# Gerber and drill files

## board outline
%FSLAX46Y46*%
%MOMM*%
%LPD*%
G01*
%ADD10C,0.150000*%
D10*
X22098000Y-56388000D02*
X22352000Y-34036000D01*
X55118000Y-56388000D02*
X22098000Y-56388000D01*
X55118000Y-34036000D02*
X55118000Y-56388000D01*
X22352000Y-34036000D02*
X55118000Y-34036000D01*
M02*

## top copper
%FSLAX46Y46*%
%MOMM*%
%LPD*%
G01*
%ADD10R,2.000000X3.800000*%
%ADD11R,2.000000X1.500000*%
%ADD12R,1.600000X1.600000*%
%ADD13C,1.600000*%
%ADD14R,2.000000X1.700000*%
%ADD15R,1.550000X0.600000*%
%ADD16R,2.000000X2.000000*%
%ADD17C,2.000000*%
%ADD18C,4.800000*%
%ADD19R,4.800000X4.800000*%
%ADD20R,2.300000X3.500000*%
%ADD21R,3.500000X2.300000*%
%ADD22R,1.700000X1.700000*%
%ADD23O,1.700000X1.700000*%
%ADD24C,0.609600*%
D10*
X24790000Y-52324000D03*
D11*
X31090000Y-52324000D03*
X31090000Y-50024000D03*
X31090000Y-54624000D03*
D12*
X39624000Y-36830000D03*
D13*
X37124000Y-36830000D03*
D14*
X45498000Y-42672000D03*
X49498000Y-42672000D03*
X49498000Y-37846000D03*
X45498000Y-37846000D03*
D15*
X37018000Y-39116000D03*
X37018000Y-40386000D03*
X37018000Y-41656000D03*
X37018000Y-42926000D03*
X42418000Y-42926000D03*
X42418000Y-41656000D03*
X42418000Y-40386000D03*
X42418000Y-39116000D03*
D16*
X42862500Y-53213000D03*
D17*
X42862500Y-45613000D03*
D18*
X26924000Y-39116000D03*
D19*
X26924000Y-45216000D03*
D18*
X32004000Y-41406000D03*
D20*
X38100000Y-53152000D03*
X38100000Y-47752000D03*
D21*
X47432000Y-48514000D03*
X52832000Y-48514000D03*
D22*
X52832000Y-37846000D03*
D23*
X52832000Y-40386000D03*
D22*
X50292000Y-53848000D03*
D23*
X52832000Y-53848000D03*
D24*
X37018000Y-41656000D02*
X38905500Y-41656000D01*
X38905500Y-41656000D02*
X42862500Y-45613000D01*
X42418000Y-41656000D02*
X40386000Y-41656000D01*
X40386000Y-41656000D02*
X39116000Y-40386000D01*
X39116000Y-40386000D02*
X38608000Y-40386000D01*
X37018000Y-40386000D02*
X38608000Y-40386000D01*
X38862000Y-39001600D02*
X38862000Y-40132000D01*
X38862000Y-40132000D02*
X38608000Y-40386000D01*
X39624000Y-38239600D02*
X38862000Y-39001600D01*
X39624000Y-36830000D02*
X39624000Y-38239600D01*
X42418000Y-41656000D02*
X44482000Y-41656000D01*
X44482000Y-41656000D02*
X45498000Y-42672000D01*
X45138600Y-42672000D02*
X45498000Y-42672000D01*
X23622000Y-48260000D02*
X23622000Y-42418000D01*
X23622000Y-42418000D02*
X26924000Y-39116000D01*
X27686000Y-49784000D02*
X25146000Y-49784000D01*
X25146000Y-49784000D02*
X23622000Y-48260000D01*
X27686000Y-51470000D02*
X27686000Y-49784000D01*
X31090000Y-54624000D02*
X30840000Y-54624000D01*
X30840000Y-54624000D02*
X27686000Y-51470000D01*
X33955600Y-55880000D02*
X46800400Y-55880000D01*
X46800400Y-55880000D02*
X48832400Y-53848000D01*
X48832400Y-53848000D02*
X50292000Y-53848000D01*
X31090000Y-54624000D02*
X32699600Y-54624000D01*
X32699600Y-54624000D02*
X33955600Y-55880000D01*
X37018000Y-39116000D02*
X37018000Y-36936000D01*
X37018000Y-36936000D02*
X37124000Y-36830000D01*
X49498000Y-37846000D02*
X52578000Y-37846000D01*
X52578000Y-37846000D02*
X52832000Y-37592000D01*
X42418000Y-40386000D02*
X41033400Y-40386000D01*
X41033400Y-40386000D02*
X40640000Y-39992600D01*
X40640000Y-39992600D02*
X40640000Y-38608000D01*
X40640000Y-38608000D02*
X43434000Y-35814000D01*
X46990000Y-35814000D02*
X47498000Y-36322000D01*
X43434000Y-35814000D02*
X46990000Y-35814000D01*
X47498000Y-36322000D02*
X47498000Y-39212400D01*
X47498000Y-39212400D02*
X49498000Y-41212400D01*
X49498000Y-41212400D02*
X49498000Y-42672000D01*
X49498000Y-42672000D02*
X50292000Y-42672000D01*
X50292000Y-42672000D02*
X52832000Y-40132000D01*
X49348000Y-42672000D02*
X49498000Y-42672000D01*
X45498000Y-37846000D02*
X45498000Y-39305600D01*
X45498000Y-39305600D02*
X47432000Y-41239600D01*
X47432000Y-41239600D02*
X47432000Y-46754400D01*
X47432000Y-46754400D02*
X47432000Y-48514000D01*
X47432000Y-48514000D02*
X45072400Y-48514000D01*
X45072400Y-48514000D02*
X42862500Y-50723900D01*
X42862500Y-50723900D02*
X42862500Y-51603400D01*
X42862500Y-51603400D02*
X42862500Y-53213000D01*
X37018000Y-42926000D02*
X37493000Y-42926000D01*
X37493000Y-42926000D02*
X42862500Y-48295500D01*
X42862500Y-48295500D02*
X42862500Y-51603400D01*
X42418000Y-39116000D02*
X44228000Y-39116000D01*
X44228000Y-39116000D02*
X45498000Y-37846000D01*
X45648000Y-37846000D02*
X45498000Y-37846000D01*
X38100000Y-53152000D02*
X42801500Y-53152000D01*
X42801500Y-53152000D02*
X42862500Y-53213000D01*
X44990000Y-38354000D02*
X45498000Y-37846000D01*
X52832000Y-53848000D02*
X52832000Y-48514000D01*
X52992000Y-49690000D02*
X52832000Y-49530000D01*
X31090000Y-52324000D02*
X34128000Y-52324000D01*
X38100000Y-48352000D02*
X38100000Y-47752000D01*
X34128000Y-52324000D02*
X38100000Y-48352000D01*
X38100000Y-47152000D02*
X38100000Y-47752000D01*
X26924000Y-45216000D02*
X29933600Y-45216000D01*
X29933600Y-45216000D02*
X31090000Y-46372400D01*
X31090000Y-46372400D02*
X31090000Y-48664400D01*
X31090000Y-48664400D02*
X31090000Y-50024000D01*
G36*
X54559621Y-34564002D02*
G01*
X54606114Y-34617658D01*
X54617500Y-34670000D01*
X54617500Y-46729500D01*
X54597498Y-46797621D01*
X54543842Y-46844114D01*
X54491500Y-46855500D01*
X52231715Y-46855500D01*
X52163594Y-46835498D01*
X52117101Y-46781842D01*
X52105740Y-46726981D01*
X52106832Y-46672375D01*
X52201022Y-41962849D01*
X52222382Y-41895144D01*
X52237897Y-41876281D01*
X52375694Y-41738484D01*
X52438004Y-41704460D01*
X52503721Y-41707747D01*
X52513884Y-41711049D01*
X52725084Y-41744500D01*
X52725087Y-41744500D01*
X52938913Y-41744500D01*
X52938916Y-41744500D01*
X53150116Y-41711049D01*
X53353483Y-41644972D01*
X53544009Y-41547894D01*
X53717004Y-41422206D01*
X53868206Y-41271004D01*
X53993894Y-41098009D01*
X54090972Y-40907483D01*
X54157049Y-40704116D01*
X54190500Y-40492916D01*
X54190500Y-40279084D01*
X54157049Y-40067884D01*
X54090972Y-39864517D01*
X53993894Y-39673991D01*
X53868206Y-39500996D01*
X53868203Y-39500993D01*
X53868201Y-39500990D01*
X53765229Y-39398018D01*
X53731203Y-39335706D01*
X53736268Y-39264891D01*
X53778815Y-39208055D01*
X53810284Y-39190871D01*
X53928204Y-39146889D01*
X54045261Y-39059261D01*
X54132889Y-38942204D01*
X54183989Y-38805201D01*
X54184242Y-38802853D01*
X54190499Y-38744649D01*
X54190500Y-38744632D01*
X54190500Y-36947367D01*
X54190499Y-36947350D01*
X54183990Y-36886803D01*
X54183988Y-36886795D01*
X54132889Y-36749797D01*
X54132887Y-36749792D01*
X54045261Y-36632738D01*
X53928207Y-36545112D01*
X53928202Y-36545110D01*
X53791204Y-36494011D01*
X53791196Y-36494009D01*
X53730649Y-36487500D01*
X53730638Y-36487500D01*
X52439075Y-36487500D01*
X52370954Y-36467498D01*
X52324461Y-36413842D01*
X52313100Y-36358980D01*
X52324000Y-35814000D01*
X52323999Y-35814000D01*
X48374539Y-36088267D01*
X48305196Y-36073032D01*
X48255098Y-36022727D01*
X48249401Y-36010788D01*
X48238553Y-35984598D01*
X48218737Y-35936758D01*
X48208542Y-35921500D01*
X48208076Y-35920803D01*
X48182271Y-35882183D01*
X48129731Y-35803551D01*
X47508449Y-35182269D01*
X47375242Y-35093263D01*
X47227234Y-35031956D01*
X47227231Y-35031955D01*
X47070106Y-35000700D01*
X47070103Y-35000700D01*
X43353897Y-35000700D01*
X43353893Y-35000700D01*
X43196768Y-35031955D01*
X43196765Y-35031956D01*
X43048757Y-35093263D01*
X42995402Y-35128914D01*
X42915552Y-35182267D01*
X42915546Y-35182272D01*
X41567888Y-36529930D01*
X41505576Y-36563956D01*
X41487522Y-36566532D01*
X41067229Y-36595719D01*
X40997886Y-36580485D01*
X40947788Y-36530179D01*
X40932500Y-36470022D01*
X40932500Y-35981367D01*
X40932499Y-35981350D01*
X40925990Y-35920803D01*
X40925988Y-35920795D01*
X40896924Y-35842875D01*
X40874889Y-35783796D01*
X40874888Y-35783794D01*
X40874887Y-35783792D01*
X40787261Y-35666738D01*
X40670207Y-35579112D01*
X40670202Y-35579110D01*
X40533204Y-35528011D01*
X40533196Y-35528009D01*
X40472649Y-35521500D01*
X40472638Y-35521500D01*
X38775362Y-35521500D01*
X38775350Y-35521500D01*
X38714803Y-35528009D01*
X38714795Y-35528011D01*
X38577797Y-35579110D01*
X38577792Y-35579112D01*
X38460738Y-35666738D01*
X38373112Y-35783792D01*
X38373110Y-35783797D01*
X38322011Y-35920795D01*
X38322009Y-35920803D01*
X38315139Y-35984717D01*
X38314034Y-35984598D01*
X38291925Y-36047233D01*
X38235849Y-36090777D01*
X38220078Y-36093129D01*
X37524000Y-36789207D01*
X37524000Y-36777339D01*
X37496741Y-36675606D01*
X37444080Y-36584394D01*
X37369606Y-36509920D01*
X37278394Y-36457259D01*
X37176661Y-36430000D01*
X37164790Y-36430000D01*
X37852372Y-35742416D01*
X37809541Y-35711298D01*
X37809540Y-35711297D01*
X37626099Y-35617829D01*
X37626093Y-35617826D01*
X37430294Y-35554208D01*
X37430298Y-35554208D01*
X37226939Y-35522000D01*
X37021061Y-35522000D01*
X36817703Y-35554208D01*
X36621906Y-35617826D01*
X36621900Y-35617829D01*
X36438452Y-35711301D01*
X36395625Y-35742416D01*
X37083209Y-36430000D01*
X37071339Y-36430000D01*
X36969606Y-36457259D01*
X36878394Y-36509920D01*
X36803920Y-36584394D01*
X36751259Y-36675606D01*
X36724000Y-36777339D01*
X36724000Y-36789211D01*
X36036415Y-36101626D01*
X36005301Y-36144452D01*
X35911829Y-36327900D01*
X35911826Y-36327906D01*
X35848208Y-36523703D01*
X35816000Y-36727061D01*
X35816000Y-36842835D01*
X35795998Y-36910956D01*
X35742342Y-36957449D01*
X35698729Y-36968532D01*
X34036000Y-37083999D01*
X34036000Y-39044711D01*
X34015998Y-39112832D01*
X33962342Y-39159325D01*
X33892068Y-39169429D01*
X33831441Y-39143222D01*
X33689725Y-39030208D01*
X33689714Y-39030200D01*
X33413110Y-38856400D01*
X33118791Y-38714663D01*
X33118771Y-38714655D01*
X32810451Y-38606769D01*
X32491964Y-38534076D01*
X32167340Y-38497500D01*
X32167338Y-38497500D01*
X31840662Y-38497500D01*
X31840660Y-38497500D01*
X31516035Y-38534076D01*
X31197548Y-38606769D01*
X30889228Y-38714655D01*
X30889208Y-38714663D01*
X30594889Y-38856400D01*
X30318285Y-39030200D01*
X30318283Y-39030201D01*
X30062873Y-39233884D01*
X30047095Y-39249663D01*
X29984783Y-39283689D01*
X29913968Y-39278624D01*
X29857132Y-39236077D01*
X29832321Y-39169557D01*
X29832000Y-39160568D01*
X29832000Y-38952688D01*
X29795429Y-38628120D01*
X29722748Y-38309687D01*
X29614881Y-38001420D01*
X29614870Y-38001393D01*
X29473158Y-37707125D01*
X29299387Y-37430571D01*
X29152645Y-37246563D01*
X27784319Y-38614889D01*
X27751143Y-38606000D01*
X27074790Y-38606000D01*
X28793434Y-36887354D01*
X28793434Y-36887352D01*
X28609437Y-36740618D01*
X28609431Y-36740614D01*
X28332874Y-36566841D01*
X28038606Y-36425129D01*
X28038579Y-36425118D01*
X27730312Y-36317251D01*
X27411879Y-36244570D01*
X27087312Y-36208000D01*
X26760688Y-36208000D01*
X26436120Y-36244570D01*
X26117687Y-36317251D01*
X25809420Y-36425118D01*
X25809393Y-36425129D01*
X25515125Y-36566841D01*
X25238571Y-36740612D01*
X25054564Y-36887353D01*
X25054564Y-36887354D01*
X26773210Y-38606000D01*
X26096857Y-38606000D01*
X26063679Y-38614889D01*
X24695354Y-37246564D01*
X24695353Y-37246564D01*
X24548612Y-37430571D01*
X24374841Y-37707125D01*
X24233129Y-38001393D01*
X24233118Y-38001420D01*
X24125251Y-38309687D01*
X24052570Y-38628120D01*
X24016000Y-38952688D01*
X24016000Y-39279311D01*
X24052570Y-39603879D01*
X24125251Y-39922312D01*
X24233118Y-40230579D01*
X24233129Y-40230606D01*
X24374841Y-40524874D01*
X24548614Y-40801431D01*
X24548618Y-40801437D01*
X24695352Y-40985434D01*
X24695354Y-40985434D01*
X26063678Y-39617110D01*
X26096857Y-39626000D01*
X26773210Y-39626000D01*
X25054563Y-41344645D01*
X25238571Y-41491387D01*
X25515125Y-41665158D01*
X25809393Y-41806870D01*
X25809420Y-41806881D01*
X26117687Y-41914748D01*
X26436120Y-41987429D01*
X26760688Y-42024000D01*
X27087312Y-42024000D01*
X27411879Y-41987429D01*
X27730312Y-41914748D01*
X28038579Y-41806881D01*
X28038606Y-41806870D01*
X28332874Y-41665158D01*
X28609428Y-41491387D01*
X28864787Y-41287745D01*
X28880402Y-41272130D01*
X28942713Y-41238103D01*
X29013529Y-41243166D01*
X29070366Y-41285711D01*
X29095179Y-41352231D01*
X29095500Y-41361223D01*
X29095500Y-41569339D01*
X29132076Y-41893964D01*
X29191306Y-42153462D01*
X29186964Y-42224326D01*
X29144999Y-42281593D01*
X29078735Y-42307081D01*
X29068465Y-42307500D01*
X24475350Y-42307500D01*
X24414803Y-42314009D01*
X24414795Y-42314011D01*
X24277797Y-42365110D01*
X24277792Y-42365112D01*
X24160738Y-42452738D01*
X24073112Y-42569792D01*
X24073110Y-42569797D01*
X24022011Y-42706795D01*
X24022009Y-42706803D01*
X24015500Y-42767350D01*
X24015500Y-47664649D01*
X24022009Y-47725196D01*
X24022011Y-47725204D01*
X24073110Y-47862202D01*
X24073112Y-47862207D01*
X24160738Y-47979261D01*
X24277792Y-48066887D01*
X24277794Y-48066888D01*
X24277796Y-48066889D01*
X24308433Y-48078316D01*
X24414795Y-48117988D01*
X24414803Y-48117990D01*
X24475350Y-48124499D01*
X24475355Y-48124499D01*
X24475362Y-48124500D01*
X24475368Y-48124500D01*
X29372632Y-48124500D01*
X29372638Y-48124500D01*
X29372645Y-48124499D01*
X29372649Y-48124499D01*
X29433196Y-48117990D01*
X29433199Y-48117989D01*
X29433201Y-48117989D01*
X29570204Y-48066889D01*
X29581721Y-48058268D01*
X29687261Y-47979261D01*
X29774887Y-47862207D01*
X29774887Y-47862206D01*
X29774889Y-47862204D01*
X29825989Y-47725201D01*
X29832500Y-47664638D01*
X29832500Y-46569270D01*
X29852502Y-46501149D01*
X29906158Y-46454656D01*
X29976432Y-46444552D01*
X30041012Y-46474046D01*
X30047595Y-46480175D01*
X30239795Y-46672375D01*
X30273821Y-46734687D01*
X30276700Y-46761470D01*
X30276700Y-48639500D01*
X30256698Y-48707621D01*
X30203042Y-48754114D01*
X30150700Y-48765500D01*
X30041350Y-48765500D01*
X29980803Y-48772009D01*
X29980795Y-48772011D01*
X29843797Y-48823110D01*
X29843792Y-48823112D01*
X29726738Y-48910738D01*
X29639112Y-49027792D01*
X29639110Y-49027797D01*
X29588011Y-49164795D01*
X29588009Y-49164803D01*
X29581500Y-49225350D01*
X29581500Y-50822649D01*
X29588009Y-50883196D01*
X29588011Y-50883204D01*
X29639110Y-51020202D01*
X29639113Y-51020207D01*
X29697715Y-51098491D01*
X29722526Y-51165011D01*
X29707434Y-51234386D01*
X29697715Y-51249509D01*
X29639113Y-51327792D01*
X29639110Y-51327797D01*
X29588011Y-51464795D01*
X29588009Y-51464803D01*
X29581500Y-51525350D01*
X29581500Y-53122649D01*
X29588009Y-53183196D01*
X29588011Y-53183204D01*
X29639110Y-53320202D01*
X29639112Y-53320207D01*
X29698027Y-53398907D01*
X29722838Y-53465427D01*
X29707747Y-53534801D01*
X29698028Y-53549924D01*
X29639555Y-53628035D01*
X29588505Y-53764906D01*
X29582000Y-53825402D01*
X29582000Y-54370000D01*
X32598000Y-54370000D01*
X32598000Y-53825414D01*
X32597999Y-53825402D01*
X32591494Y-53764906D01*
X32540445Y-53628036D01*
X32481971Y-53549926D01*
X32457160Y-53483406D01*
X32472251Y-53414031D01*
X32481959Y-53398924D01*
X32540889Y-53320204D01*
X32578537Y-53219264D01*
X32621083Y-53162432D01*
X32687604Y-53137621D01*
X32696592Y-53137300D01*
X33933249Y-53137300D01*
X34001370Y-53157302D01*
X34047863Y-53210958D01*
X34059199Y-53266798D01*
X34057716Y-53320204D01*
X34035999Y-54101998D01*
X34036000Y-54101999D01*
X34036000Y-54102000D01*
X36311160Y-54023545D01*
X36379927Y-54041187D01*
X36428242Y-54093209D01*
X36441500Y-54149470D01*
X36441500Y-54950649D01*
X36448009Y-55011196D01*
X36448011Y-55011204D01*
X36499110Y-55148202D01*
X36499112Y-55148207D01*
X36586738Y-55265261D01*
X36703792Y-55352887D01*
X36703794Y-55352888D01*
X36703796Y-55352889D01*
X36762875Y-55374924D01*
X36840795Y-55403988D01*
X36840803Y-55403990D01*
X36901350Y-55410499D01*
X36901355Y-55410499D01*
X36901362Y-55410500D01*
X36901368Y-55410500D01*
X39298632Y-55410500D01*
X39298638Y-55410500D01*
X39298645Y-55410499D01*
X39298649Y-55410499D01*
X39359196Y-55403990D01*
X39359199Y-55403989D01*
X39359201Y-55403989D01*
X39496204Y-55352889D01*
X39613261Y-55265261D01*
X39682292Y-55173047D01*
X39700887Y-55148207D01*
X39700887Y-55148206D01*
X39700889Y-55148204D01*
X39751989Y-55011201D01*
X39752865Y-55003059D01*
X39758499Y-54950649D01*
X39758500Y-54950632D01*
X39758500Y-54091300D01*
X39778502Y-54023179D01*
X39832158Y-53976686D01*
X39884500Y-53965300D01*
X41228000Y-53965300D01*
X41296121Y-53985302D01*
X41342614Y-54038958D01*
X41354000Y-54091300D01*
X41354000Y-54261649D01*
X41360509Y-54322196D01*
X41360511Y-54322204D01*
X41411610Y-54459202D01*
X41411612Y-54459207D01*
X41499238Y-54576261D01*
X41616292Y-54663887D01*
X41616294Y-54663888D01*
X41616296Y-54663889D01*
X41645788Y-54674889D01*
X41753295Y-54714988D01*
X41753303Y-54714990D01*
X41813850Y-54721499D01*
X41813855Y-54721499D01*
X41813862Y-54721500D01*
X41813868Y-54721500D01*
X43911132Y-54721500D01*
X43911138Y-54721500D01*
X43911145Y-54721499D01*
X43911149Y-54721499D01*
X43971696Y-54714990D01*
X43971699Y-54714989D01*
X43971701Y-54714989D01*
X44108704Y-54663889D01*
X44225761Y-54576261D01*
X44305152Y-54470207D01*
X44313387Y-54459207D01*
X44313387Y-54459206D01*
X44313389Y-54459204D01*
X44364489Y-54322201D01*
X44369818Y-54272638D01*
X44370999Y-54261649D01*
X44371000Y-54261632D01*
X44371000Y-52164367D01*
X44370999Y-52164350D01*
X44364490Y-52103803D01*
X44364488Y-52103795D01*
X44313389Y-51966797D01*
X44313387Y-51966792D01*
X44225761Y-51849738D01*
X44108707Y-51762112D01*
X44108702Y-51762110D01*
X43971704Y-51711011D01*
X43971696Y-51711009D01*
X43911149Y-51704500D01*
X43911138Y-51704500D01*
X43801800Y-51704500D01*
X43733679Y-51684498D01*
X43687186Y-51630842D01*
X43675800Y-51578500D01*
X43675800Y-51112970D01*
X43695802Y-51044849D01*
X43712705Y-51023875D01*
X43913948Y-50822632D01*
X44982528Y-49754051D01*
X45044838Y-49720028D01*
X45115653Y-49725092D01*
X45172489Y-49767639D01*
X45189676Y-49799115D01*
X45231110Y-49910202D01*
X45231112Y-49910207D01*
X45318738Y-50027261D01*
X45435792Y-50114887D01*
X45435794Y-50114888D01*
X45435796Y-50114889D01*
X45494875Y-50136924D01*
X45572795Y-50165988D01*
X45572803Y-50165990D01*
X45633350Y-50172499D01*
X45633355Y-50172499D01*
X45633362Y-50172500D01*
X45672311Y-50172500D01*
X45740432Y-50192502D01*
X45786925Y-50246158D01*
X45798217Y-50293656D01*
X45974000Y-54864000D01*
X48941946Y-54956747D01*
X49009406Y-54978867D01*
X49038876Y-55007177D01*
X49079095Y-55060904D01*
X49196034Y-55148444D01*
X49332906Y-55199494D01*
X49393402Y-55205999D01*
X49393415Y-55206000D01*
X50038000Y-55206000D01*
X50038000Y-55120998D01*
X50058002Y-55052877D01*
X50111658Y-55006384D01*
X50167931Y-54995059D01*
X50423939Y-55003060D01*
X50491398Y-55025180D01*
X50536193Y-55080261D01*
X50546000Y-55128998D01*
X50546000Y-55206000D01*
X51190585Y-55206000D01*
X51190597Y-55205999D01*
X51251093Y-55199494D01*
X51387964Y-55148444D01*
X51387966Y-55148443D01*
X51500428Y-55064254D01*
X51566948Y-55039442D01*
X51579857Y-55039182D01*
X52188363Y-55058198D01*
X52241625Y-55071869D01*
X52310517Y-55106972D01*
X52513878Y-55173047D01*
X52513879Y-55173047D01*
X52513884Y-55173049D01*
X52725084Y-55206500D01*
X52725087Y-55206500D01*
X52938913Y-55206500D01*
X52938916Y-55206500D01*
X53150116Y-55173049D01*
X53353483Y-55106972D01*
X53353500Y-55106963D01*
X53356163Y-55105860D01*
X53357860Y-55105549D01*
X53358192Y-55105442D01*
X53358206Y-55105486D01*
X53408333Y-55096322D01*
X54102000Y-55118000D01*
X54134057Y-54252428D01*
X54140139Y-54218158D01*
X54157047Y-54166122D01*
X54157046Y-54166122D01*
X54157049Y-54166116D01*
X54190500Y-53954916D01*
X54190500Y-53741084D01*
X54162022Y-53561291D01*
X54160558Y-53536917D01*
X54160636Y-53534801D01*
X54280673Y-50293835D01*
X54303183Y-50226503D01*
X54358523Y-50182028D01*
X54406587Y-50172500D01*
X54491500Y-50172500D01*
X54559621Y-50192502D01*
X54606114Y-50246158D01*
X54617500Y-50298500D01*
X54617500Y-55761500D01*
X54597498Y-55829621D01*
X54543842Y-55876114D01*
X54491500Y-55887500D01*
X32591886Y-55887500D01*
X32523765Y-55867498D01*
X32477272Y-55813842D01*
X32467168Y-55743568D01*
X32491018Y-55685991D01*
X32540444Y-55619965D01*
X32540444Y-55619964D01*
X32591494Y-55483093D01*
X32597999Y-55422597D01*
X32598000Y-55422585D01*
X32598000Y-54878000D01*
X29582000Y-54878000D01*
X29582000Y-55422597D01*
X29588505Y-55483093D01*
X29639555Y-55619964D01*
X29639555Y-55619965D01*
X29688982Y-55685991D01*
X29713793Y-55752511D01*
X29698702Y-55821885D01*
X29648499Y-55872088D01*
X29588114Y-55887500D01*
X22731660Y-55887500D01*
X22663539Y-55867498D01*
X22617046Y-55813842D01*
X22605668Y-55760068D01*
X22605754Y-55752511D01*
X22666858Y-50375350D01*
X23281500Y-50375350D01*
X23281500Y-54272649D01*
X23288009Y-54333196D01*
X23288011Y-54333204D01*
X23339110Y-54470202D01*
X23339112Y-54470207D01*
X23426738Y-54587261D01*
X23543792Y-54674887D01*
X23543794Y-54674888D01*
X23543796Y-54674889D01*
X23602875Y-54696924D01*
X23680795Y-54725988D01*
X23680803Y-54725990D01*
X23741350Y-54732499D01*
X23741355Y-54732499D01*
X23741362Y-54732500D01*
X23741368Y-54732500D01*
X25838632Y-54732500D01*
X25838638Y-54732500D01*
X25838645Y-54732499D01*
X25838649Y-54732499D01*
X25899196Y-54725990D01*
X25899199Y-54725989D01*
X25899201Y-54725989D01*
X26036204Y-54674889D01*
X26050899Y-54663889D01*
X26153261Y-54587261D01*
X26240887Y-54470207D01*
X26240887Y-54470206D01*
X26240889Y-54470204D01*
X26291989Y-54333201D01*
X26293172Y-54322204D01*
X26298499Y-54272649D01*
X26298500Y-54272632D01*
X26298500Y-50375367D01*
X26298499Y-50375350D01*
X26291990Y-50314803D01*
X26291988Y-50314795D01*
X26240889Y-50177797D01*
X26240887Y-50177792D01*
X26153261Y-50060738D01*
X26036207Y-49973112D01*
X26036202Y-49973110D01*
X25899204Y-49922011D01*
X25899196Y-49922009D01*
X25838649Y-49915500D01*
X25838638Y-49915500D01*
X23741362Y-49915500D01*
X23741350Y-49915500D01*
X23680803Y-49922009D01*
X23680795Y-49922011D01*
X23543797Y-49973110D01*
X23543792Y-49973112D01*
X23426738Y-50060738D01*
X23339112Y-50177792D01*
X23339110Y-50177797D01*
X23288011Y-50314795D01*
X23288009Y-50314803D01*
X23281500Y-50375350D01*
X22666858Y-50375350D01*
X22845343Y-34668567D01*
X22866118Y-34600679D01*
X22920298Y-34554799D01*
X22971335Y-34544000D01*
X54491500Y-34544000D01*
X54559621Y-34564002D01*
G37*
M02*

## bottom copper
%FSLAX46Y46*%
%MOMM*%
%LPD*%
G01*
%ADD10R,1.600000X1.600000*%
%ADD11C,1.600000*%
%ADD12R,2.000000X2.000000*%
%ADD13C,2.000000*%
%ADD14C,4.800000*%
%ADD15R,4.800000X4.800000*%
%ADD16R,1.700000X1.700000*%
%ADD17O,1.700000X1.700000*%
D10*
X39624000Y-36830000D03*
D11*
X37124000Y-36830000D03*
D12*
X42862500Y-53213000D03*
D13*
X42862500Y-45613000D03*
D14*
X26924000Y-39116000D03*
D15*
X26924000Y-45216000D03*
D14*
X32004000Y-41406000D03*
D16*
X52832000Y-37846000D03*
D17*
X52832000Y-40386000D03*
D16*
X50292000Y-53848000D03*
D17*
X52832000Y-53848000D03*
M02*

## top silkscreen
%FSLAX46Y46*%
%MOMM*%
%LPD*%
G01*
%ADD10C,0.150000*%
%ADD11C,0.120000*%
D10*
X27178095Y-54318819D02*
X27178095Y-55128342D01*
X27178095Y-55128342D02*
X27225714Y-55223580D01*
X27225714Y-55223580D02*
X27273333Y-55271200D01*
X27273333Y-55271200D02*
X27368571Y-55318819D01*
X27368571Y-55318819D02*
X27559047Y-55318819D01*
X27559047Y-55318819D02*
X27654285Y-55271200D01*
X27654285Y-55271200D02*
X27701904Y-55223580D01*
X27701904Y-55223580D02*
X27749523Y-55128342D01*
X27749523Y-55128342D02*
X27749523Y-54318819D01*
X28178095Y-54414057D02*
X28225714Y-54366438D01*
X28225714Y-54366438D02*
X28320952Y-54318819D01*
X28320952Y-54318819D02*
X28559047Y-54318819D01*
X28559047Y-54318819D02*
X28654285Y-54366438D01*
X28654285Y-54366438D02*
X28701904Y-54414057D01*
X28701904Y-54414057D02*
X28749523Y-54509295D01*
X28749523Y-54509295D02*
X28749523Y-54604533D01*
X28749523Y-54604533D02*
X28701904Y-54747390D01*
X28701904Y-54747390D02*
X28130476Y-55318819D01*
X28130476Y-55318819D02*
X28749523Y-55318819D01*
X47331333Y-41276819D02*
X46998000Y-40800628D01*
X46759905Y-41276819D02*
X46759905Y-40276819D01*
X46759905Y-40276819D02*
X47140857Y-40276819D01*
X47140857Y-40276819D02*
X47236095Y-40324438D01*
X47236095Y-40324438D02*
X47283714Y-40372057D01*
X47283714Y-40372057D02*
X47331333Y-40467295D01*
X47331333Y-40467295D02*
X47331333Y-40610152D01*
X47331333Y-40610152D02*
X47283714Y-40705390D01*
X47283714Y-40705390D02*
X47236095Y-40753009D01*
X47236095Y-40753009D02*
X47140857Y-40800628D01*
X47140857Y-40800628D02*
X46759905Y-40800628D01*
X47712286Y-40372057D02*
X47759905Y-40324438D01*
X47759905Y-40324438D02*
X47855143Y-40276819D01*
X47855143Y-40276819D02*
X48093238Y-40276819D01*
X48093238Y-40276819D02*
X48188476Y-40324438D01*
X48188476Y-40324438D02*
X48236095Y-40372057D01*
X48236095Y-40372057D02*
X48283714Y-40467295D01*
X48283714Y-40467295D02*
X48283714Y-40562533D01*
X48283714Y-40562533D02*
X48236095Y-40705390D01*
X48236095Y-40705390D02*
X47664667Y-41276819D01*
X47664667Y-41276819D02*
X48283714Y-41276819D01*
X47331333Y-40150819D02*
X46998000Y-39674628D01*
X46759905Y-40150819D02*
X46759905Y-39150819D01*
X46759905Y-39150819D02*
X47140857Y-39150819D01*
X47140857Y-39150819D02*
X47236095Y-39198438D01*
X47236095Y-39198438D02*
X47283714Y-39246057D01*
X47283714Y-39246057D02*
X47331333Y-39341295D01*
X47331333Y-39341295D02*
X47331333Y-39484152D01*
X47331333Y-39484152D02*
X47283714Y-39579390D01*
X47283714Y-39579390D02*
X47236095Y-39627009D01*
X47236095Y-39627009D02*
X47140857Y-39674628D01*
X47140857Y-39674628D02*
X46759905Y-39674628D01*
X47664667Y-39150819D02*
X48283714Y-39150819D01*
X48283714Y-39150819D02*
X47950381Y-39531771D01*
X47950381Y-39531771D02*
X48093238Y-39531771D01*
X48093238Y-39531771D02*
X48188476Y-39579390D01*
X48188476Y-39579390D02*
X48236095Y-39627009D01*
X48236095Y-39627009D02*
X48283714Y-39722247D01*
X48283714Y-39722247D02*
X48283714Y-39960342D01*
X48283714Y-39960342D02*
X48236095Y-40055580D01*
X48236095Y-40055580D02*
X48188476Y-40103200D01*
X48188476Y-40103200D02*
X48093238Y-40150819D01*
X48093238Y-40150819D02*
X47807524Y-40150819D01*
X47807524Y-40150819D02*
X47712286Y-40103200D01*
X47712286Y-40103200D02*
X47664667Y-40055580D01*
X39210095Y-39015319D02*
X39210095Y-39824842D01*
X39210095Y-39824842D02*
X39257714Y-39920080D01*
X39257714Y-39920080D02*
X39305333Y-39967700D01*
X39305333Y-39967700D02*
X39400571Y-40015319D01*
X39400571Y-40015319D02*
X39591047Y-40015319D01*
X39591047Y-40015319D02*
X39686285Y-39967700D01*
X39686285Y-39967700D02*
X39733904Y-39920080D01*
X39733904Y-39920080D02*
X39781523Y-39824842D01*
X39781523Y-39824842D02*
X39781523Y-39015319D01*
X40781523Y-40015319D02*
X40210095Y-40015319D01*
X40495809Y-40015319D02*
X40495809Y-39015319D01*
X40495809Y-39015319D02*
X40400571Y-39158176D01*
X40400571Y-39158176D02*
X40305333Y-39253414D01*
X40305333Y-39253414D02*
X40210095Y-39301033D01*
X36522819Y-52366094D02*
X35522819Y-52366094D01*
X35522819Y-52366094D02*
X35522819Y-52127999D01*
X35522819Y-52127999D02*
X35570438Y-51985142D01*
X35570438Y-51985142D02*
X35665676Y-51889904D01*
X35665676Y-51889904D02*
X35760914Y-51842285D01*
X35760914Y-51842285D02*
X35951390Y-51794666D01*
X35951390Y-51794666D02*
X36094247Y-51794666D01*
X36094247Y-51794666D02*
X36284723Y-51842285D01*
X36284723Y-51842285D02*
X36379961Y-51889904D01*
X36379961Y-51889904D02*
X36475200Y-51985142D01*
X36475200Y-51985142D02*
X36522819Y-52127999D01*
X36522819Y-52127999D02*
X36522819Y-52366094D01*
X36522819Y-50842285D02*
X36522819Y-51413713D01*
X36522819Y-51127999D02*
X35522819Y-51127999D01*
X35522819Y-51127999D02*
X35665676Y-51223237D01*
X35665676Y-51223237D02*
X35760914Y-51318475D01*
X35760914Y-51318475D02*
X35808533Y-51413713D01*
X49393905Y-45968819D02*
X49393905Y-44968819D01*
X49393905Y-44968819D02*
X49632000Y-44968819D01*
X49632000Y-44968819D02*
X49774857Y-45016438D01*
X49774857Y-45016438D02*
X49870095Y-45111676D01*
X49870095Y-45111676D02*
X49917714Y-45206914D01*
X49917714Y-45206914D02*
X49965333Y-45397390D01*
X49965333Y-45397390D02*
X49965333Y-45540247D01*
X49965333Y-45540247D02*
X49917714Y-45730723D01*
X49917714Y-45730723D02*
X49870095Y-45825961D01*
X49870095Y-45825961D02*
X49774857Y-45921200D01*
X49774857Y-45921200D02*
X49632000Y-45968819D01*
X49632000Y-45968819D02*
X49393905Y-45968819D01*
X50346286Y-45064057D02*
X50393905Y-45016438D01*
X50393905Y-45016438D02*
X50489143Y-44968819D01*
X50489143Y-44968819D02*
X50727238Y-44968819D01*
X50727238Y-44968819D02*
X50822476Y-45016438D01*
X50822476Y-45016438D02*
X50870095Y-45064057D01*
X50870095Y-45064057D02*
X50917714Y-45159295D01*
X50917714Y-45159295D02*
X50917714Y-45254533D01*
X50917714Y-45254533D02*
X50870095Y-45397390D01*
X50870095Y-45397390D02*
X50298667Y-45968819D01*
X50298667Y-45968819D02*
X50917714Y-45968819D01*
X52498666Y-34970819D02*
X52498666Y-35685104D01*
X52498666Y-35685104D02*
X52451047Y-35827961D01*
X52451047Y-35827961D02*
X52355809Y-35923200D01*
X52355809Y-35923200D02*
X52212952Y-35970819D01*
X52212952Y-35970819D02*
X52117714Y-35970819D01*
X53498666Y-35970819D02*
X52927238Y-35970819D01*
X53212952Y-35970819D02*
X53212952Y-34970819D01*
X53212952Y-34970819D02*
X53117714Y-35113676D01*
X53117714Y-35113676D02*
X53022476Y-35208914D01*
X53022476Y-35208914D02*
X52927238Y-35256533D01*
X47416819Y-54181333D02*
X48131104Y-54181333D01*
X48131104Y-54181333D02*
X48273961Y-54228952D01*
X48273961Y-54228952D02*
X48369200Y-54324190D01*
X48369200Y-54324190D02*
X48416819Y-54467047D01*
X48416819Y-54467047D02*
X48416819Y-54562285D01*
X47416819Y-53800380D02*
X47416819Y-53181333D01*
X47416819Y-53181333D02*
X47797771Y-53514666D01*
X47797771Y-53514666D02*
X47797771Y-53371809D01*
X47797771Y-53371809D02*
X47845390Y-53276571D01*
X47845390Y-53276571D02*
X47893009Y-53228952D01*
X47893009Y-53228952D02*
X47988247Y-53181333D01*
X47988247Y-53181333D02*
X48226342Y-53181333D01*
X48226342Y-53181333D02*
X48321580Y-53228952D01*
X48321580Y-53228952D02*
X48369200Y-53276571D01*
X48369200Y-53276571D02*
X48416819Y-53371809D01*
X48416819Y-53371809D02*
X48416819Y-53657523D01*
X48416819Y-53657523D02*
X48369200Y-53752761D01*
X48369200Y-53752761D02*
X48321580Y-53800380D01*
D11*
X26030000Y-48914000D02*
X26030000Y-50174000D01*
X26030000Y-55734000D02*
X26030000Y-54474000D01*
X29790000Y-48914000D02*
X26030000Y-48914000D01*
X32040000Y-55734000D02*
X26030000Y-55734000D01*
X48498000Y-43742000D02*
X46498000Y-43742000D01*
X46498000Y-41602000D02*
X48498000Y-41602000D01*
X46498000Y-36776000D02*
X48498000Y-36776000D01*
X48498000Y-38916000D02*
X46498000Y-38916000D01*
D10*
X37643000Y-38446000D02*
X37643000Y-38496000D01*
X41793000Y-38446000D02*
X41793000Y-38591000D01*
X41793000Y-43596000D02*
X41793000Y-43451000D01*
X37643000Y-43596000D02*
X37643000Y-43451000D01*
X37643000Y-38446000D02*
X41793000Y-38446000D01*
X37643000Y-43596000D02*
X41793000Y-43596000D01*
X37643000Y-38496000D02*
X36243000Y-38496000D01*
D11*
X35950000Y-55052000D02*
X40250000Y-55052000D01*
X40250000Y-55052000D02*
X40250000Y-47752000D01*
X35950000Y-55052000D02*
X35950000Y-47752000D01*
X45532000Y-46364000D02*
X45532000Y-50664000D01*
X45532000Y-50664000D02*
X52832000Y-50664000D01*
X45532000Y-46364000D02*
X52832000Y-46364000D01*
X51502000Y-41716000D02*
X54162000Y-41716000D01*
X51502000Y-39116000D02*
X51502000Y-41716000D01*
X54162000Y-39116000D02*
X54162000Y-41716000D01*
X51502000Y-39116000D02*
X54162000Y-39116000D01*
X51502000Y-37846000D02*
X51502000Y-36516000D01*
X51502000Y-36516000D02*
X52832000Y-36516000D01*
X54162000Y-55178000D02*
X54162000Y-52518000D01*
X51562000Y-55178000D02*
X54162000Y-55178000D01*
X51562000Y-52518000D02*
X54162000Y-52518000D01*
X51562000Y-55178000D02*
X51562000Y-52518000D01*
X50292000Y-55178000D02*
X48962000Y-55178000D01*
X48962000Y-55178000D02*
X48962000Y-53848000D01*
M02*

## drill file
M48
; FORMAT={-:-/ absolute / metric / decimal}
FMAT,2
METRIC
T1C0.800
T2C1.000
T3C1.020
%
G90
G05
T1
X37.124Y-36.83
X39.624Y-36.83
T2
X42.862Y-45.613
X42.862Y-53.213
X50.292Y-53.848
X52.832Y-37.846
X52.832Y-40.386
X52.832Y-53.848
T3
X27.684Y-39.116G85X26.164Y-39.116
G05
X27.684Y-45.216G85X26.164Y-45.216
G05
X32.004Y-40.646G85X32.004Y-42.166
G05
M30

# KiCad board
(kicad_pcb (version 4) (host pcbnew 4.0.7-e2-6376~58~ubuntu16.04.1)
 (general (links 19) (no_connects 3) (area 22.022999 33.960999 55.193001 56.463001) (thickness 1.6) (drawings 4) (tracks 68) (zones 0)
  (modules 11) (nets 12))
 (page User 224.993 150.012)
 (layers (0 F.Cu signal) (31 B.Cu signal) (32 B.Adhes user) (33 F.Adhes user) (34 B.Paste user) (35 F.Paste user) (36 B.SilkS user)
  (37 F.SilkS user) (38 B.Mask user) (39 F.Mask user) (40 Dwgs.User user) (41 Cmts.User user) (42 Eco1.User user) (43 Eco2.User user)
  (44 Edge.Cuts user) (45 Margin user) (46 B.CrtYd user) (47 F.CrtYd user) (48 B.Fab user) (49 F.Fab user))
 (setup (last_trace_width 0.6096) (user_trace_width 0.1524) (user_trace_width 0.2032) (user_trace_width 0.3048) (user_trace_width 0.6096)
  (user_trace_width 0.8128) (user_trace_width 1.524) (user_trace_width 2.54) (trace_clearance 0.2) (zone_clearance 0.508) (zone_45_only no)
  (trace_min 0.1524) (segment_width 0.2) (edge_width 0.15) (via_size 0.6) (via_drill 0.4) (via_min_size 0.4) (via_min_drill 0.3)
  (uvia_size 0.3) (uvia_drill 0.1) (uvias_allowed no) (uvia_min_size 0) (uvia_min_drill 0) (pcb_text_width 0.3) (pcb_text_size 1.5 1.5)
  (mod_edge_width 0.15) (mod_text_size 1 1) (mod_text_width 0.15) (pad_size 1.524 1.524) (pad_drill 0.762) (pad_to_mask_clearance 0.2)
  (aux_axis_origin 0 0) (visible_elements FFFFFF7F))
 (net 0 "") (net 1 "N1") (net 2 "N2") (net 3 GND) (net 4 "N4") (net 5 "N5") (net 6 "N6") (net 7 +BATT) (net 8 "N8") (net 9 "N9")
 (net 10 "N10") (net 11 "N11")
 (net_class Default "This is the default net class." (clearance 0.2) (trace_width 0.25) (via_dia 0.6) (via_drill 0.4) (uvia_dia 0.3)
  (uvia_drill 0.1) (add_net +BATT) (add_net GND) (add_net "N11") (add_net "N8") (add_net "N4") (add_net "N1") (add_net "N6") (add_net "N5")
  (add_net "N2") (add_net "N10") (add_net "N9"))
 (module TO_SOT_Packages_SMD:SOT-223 (layer F.Cu) (at 27.94 52.324 180)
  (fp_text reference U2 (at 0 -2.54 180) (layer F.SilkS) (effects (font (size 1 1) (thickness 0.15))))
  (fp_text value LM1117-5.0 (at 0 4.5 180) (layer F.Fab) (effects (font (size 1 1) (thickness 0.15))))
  (fp_line (start 1.91 3.41) (end 1.91 2.15) (layer F.SilkS) (width 0.12))
  (fp_line (start 1.91 -3.41) (end 1.91 -2.15) (layer F.SilkS) (width 0.12))
  (fp_line (start -1.85 3.41) (end 1.91 3.41) (layer F.SilkS) (width 0.12))
  (fp_line (start -4.1 -3.41) (end 1.91 -3.41) (layer F.SilkS) (width 0.12))
  (pad 4 smd rect (at 3.15 0 180) (size 2 3.8) (layers F.Cu F.Paste F.Mask))
  (pad 2 smd rect (at -3.15 0 180) (size 2 1.5) (layers F.Cu F.Paste F.Mask) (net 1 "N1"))
  (pad 3 smd rect (at -3.15 2.3 180) (size 2 1.5) (layers F.Cu F.Paste F.Mask) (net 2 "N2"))
  (pad 1 smd rect (at -3.15 -2.3 180) (size 2 1.5) (layers F.Cu F.Paste F.Mask) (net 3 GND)))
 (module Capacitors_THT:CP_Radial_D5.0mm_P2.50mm (layer B.Cu) (at 39.624 36.83 180)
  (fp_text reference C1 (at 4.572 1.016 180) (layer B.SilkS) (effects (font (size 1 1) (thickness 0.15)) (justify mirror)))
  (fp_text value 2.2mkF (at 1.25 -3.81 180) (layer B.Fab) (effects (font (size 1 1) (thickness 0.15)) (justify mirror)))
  (pad 1 thru_hole rect (at 0 0 180) (size 1.6 1.6) (drill 0.8) (layers *.Cu *.Mask) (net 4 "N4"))
  (pad 2 thru_hole circle (at 2.5 0 180) (size 1.6 1.6) (drill 0.8) (layers *.Cu *.Mask) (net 3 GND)))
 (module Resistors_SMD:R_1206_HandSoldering (layer F.Cu) (at 47.498 42.672)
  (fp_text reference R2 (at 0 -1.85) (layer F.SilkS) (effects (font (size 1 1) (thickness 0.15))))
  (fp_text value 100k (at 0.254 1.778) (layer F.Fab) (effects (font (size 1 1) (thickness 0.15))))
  (fp_line (start 1 1.07) (end -1 1.07) (layer F.SilkS) (width 0.12))
  (fp_line (start -1 -1.07) (end 1 -1.07) (layer F.SilkS) (width 0.12))
  (pad 1 smd rect (at -2 0) (size 2 1.7) (layers F.Cu F.Paste F.Mask) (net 4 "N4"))
  (pad 2 smd rect (at 2 0) (size 2 1.7) (layers F.Cu F.Paste F.Mask) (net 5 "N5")))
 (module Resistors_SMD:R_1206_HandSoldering (layer F.Cu) (at 47.498 37.846 180)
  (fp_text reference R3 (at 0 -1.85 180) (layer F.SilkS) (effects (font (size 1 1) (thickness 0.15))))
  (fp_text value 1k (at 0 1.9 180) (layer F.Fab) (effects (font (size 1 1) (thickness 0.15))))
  (fp_line (start 1 1.07) (end -1 1.07) (layer F.SilkS) (width 0.12))
  (fp_line (start -1 -1.07) (end 1 -1.07) (layer F.SilkS) (width 0.12))
  (pad 1 smd rect (at -2 0 180) (size 2 1.7) (layers F.Cu F.Paste F.Mask) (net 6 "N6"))
  (pad 2 smd rect (at 2 0 180) (size 2 1.7) (layers F.Cu F.Paste F.Mask) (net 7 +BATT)))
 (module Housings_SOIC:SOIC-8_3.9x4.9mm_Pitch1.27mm (layer F.Cu) (at 39.718 41.021)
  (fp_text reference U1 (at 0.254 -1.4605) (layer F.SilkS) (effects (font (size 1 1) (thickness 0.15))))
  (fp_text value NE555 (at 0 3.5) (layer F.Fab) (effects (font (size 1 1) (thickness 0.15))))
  (fp_line (start -2.075 -2.575) (end -2.075 -2.525) (layer F.SilkS) (width 0.15))
  (fp_line (start 2.075 -2.575) (end 2.075 -2.43) (layer F.SilkS) (width 0.15))
  (fp_line (start 2.075 2.575) (end 2.075 2.43) (layer F.SilkS) (width 0.15))
  (fp_line (start -2.075 2.575) (end -2.075 2.43) (layer F.SilkS) (width 0.15))
  (fp_line (start -2.075 -2.575) (end 2.075 -2.575) (layer F.SilkS) (width 0.15))
  (fp_line (start -2.075 2.575) (end 2.075 2.575) (layer F.SilkS) (width 0.15))
  (fp_line (start -2.075 -2.525) (end -3.475 -2.525) (layer F.SilkS) (width 0.15))
  (pad 1 smd rect (at -2.7 -1.905) (size 1.55 0.6) (layers F.Cu F.Paste F.Mask) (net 3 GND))
  (pad 2 smd rect (at -2.7 -0.635) (size 1.55 0.6) (layers F.Cu F.Paste F.Mask) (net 4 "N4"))
  (pad 3 smd rect (at -2.7 0.635) (size 1.55 0.6) (layers F.Cu F.Paste F.Mask) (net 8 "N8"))
  (pad 4 smd rect (at -2.7 1.905) (size 1.55 0.6) (layers F.Cu F.Paste F.Mask) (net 7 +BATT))
  (pad 5 smd rect (at 2.7 1.905) (size 1.55 0.6) (layers F.Cu F.Paste F.Mask) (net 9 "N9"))
  (pad 6 smd rect (at 2.7 0.635) (size 1.55 0.6) (layers F.Cu F.Paste F.Mask) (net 4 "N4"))
  (pad 7 smd rect (at 2.7 -0.635) (size 1.55 0.6) (layers F.Cu F.Paste F.Mask) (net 5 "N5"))
  (pad 8 smd rect (at 2.7 -1.905) (size 1.55 0.6) (layers F.Cu F.Paste F.Mask) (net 7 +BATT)))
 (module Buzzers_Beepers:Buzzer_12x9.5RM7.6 (layer B.Cu) (at 42.8625 53.213 90)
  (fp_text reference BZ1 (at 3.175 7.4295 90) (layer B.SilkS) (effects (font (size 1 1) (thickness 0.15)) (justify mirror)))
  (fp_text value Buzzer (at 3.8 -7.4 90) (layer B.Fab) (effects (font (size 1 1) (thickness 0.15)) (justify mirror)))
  (pad 1 thru_hole rect (at 0 0 90) (size 2 2) (drill 1) (layers *.Cu *.Mask) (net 7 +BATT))
  (pad 2 thru_hole circle (at 7.6 0 90) (size 2 2) (drill 1) (layers *.Cu *.Mask) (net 8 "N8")))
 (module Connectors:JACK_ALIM (layer B.Cu) (at 26.924 45.216 270)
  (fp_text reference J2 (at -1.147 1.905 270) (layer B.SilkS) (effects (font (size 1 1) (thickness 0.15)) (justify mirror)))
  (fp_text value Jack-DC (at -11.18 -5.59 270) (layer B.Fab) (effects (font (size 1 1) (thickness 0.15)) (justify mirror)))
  (pad 2 thru_hole circle (at -6.1 0 270) (size 4.8 4.8) (drill oval 1.02 2.54) (layers *.Cu *.Mask) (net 3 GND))
  (pad 1 thru_hole rect (at 0 0 270) (size 4.8 4.8) (drill oval 1.02 2.54) (layers *.Cu *.Mask) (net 2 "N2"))
  (pad 3 thru_hole circle (at -3.81 -5.08 270) (size 4.8 4.8) (drill oval 2.54 1.02) (layers *.Cu *.Mask) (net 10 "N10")))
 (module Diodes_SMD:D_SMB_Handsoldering (layer F.Cu) (at 38.1 50.452 90)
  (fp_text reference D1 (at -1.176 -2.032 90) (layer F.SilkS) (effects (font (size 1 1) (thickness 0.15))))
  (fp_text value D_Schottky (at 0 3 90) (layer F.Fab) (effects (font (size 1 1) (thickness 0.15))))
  (fp_line (start -4.6 -2.15) (end -4.6 2.15) (layer F.SilkS) (width 0.12))
  (fp_line (start -4.6 2.15) (end 2.7 2.15) (layer F.SilkS) (width 0.12))
  (fp_line (start -4.6 -2.15) (end 2.7 -2.15) (layer F.SilkS) (width 0.12))
  (pad 1 smd rect (at -2.7 0 90) (size 3.5 2.3) (layers F.Cu F.Paste F.Mask) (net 7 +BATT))
  (pad 2 smd rect (at 2.7 0 90) (size 3.5 2.3) (layers F.Cu F.Paste F.Mask) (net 1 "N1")))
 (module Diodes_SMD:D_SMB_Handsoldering (layer F.Cu) (at 50.132 48.514)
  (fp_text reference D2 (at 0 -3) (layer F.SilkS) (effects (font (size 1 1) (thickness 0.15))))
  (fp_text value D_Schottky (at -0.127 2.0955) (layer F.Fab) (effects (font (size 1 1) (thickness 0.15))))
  (fp_line (start -4.6 -2.15) (end -4.6 2.15) (layer F.SilkS) (width 0.12))
  (fp_line (start -4.6 2.15) (end 2.7 2.15) (layer F.SilkS) (width 0.12))
  (fp_line (start -4.6 -2.15) (end 2.7 -2.15) (layer F.SilkS) (width 0.12))
  (pad 1 smd rect (at -2.7 0) (size 3.5 2.3) (layers F.Cu F.Paste F.Mask) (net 7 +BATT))
  (pad 2 smd rect (at 2.7 0) (size 3.5 2.3) (layers F.Cu F.Paste F.Mask) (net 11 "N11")))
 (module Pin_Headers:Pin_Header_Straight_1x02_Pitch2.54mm (layer F.Cu) (at 52.832 37.846)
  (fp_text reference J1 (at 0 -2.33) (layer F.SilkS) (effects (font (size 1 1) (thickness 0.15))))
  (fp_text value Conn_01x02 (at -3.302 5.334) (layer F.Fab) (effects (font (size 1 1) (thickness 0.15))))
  (fp_line (start -1.33 3.87) (end 1.33 3.87) (layer F.SilkS) (width 0.12))
  (fp_line (start -1.33 1.27) (end -1.33 3.87) (layer F.SilkS) (width 0.12))
  (fp_line (start 1.33 1.27) (end 1.33 3.87) (layer F.SilkS) (width 0.12))
  (fp_line (start -1.33 1.27) (end 1.33 1.27) (layer F.SilkS) (width 0.12))
  (fp_line (start -1.33 0) (end -1.33 -1.33) (layer F.SilkS) (width 0.12))
  (fp_line (start -1.33 -1.33) (end 0 -1.33) (layer F.SilkS) (width 0.12))
  (pad 1 thru_hole rect (at 0 0) (size 1.7 1.7) (drill 1) (layers *.Cu *.Mask) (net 6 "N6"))
  (pad 2 thru_hole oval (at 0 2.54) (size 1.7 1.7) (drill 1) (layers *.Cu *.Mask) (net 5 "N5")))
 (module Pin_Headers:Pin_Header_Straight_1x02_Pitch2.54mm (layer F.Cu) (at 50.292 53.848 90)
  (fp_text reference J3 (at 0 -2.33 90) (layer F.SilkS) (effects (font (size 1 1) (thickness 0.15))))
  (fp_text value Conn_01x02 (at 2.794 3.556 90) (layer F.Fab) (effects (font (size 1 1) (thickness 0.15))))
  (fp_line (start -1.33 3.87) (end 1.33 3.87) (layer F.SilkS) (width 0.12))
  (fp_line (start -1.33 1.27) (end -1.33 3.87) (layer F.SilkS) (width 0.12))
  (fp_line (start 1.33 1.27) (end 1.33 3.87) (layer F.SilkS) (width 0.12))
  (fp_line (start -1.33 1.27) (end 1.33 1.27) (layer F.SilkS) (width 0.12))
  (fp_line (start -1.33 0) (end -1.33 -1.33) (layer F.SilkS) (width 0.12))
  (fp_line (start -1.33 -1.33) (end 0 -1.33) (layer F.SilkS) (width 0.12))
  (pad 1 thru_hole rect (at 0 0 90) (size 1.7 1.7) (drill 1) (layers *.Cu *.Mask) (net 3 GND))
  (pad 2 thru_hole oval (at 0 2.54 90) (size 1.7 1.7) (drill 1) (layers *.Cu *.Mask) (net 11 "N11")))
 (gr_line (start 22.098 56.388) (end 22.352 34.036) (layer Edge.Cuts) (width 0.15))
 (gr_line (start 55.118 56.388) (end 22.098 56.388) (layer Edge.Cuts) (width 0.15))
 (gr_line (start 55.118 34.036) (end 55.118 56.388) (layer Edge.Cuts) (width 0.15))
 (gr_line (start 22.352 34.036) (end 55.118 34.036) (layer Edge.Cuts) (width 0.15))
 (segment (start 37.018 41.656) (end 38.9055 41.656) (width 0.6096) (layer F.Cu) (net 8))
 (segment (start 38.9055 41.656) (end 42.8625 45.613) (width 0.6096) (layer F.Cu) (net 8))
 (segment (start 42.418 41.656) (end 40.386 41.656) (width 0.6096) (layer F.Cu) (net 4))
 (segment (start 40.386 41.656) (end 39.116 40.386) (width 0.6096) (layer F.Cu) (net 4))
 (segment (start 39.116 40.386) (end 38.608 40.386) (width 0.6096) (layer F.Cu) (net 4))
 (segment (start 37.018 40.386) (end 38.608 40.386) (width 0.6096) (layer F.Cu) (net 4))
 (segment (start 38.862 39.0016) (end 38.862 40.132) (width 0.6096) (layer F.Cu) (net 4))
 (segment (start 38.862 40.132) (end 38.608 40.386) (width 0.6096) (layer F.Cu) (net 4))
 (segment (start 39.624 38.2396) (end 38.862 39.0016) (width 0.6096) (layer F.Cu) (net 4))
 (segment (start 39.624 36.83) (end 39.624 38.2396) (width 0.6096) (layer F.Cu) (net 4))
 (segment (start 42.418 41.656) (end 44.482 41.656) (width 0.6096) (layer F.Cu) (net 4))
 (segment (start 44.482 41.656) (end 45.498 42.672) (width 0.6096) (layer F.Cu) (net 4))
 (segment (start 45.1386 42.672) (end 45.498 42.672) (width 0.6096) (layer F.Cu) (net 4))
 (segment (start 23.622 48.26) (end 23.622 42.418) (width 0.6096) (layer F.Cu) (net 3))
 (segment (start 23.622 42.418) (end 26.924 39.116) (width 0.6096) (layer F.Cu) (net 3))
 (segment (start 27.686 49.784) (end 25.146 49.784) (width 0.6096) (layer F.Cu) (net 3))
 (segment (start 25.146 49.784) (end 23.622 48.26) (width 0.6096) (layer F.Cu) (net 3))
 (segment (start 27.686 51.47) (end 27.686 49.784) (width 0.6096) (layer F.Cu) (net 3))
 (segment (start 31.09 54.624) (end 30.84 54.624) (width 0.6096) (layer F.Cu) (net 3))
 (segment (start 30.84 54.624) (end 27.686 51.47) (width 0.6096) (layer F.Cu) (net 3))
 (segment (start 33.9556 55.88) (end 46.8004 55.88) (width 0.6096) (layer F.Cu) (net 3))
 (segment (start 46.8004 55.88) (end 48.8324 53.848) (width 0.6096) (layer F.Cu) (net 3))
 (segment (start 48.8324 53.848) (end 50.292 53.848) (width 0.6096) (layer F.Cu) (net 3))
 (segment (start 31.09 54.624) (end 32.6996 54.624) (width 0.6096) (layer F.Cu) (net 3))
 (segment (start 32.6996 54.624) (end 33.9556 55.88) (width 0.6096) (layer F.Cu) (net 3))
 (segment (start 37.018 39.116) (end 37.018 36.936) (width 0.6096) (layer F.Cu) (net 3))
 (segment (start 37.018 36.936) (end 37.124 36.83) (width 0.6096) (layer F.Cu) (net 3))
 (segment (start 49.498 37.846) (end 52.578 37.846) (width 0.6096) (layer F.Cu) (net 6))
 (segment (start 52.578 37.846) (end 52.832 37.592) (width 0.6096) (layer F.Cu) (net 6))
 (segment (start 42.418 40.386) (end 41.0334 40.386) (width 0.6096) (layer F.Cu) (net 5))
 (segment (start 41.0334 40.386) (end 40.64 39.9926) (width 0.6096) (layer F.Cu) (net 5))
 (segment (start 40.64 39.9926) (end 40.64 38.608) (width 0.6096) (layer F.Cu) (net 5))
 (segment (start 40.64 38.608) (end 43.434 35.814) (width 0.6096) (layer F.Cu) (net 5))
 (segment (start 46.99 35.814) (end 47.498 36.322) (width 0.6096) (layer F.Cu) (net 5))
 (segment (start 43.434 35.814) (end 46.99 35.814) (width 0.6096) (layer F.Cu) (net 5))
 (segment (start 47.498 36.322) (end 47.498 39.2124) (width 0.6096) (layer F.Cu) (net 5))
 (segment (start 47.498 39.2124) (end 49.498 41.2124) (width 0.6096) (layer F.Cu) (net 5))
 (segment (start 49.498 41.2124) (end 49.498 42.672) (width 0.6096) (layer F.Cu) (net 5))
 (segment (start 49.498 42.672) (end 50.292 42.672) (width 0.6096) (layer F.Cu) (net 5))
 (segment (start 50.292 42.672) (end 52.832 40.132) (width 0.6096) (layer F.Cu) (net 5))
 (segment (start 49.348 42.672) (end 49.498 42.672) (width 0.6096) (layer F.Cu) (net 5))
 (segment (start 45.498 37.846) (end 45.498 39.3056) (width 0.6096) (layer F.Cu) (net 7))
 (segment (start 45.498 39.3056) (end 47.432 41.2396) (width 0.6096) (layer F.Cu) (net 7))
 (segment (start 47.432 41.2396) (end 47.432 46.7544) (width 0.6096) (layer F.Cu) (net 7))
 (segment (start 47.432 46.7544) (end 47.432 48.514) (width 0.6096) (layer F.Cu) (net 7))
 (segment (start 47.432 48.514) (end 45.0724 48.514) (width 0.6096) (layer F.Cu) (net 7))
 (segment (start 45.0724 48.514) (end 42.8625 50.7239) (width 0.6096) (layer F.Cu) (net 7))
 (segment (start 42.8625 50.7239) (end 42.8625 51.6034) (width 0.6096) (layer F.Cu) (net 7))
 (segment (start 42.8625 51.6034) (end 42.8625 53.213) (width 0.6096) (layer F.Cu) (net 7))
 (segment (start 37.018 42.926) (end 37.493 42.926) (width 0.6096) (layer F.Cu) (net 7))
 (segment (start 37.493 42.926) (end 42.8625 48.2955) (width 0.6096) (layer F.Cu) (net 7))
 (segment (start 42.8625 48.2955) (end 42.8625 51.6034) (width 0.6096) (layer F.Cu) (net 7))
 (segment (start 42.418 39.116) (end 44.228 39.116) (width 0.6096) (layer F.Cu) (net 7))
 (segment (start 44.228 39.116) (end 45.498 37.846) (width 0.6096) (layer F.Cu) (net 7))
 (segment (start 45.648 37.846) (end 45.498 37.846) (width 0.6096) (layer F.Cu) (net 7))
 (segment (start 38.1 53.152) (end 42.8015 53.152) (width 0.6096) (layer F.Cu) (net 7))
 (segment (start 42.8015 53.152) (end 42.8625 53.213) (width 0.6096) (layer F.Cu) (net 7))
 (segment (start 44.99 38.354) (end 45.498 37.846) (width 0.6096) (layer F.Cu) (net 7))
 (segment (start 52.832 53.848) (end 52.832 48.514) (width 0.6096) (layer F.Cu) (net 11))
 (segment (start 52.992 49.69) (end 52.832 49.53) (width 0.6096) (layer F.Cu) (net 11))
 (segment (start 31.09 52.324) (end 34.128 52.324) (width 0.6096) (layer F.Cu) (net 1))
 (segment (start 38.1 48.352) (end 38.1 47.752) (width 0.6096) (layer F.Cu) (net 1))
 (segment (start 34.128 52.324) (end 38.1 48.352) (width 0.6096) (layer F.Cu) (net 1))
 (segment (start 38.1 47.152) (end 38.1 47.752) (width 0.6096) (layer F.Cu) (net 1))
 (segment (start 26.924 45.216) (end 29.9336 45.216) (width 0.6096) (layer F.Cu) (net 2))
 (segment (start 29.9336 45.216) (end 31.09 46.3724) (width 0.6096) (layer F.Cu) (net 2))
 (segment (start 31.09 46.3724) (end 31.09 48.6644) (width 0.6096) (layer F.Cu) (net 2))
 (segment (start 31.09 48.6644) (end 31.09 50.024) (width 0.6096) (layer F.Cu) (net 2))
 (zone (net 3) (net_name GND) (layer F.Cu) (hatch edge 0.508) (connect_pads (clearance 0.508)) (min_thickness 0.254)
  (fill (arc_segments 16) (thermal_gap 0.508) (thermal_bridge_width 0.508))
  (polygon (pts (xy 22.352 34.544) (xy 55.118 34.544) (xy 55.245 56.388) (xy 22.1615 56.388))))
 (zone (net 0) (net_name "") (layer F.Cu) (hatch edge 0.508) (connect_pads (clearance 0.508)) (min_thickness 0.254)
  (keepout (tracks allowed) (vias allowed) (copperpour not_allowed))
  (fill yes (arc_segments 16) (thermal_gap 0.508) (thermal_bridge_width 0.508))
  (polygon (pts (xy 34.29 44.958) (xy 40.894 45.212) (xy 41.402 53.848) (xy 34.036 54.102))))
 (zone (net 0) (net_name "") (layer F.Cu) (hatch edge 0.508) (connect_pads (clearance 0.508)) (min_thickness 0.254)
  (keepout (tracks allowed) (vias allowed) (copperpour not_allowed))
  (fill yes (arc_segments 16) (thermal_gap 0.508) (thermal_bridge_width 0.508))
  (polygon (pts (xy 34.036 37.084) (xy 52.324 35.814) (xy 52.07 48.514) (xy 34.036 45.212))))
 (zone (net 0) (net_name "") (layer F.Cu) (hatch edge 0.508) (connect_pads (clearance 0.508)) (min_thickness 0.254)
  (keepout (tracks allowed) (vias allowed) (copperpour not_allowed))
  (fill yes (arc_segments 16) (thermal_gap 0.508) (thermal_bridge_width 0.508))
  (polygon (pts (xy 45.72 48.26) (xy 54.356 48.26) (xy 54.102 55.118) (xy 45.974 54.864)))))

